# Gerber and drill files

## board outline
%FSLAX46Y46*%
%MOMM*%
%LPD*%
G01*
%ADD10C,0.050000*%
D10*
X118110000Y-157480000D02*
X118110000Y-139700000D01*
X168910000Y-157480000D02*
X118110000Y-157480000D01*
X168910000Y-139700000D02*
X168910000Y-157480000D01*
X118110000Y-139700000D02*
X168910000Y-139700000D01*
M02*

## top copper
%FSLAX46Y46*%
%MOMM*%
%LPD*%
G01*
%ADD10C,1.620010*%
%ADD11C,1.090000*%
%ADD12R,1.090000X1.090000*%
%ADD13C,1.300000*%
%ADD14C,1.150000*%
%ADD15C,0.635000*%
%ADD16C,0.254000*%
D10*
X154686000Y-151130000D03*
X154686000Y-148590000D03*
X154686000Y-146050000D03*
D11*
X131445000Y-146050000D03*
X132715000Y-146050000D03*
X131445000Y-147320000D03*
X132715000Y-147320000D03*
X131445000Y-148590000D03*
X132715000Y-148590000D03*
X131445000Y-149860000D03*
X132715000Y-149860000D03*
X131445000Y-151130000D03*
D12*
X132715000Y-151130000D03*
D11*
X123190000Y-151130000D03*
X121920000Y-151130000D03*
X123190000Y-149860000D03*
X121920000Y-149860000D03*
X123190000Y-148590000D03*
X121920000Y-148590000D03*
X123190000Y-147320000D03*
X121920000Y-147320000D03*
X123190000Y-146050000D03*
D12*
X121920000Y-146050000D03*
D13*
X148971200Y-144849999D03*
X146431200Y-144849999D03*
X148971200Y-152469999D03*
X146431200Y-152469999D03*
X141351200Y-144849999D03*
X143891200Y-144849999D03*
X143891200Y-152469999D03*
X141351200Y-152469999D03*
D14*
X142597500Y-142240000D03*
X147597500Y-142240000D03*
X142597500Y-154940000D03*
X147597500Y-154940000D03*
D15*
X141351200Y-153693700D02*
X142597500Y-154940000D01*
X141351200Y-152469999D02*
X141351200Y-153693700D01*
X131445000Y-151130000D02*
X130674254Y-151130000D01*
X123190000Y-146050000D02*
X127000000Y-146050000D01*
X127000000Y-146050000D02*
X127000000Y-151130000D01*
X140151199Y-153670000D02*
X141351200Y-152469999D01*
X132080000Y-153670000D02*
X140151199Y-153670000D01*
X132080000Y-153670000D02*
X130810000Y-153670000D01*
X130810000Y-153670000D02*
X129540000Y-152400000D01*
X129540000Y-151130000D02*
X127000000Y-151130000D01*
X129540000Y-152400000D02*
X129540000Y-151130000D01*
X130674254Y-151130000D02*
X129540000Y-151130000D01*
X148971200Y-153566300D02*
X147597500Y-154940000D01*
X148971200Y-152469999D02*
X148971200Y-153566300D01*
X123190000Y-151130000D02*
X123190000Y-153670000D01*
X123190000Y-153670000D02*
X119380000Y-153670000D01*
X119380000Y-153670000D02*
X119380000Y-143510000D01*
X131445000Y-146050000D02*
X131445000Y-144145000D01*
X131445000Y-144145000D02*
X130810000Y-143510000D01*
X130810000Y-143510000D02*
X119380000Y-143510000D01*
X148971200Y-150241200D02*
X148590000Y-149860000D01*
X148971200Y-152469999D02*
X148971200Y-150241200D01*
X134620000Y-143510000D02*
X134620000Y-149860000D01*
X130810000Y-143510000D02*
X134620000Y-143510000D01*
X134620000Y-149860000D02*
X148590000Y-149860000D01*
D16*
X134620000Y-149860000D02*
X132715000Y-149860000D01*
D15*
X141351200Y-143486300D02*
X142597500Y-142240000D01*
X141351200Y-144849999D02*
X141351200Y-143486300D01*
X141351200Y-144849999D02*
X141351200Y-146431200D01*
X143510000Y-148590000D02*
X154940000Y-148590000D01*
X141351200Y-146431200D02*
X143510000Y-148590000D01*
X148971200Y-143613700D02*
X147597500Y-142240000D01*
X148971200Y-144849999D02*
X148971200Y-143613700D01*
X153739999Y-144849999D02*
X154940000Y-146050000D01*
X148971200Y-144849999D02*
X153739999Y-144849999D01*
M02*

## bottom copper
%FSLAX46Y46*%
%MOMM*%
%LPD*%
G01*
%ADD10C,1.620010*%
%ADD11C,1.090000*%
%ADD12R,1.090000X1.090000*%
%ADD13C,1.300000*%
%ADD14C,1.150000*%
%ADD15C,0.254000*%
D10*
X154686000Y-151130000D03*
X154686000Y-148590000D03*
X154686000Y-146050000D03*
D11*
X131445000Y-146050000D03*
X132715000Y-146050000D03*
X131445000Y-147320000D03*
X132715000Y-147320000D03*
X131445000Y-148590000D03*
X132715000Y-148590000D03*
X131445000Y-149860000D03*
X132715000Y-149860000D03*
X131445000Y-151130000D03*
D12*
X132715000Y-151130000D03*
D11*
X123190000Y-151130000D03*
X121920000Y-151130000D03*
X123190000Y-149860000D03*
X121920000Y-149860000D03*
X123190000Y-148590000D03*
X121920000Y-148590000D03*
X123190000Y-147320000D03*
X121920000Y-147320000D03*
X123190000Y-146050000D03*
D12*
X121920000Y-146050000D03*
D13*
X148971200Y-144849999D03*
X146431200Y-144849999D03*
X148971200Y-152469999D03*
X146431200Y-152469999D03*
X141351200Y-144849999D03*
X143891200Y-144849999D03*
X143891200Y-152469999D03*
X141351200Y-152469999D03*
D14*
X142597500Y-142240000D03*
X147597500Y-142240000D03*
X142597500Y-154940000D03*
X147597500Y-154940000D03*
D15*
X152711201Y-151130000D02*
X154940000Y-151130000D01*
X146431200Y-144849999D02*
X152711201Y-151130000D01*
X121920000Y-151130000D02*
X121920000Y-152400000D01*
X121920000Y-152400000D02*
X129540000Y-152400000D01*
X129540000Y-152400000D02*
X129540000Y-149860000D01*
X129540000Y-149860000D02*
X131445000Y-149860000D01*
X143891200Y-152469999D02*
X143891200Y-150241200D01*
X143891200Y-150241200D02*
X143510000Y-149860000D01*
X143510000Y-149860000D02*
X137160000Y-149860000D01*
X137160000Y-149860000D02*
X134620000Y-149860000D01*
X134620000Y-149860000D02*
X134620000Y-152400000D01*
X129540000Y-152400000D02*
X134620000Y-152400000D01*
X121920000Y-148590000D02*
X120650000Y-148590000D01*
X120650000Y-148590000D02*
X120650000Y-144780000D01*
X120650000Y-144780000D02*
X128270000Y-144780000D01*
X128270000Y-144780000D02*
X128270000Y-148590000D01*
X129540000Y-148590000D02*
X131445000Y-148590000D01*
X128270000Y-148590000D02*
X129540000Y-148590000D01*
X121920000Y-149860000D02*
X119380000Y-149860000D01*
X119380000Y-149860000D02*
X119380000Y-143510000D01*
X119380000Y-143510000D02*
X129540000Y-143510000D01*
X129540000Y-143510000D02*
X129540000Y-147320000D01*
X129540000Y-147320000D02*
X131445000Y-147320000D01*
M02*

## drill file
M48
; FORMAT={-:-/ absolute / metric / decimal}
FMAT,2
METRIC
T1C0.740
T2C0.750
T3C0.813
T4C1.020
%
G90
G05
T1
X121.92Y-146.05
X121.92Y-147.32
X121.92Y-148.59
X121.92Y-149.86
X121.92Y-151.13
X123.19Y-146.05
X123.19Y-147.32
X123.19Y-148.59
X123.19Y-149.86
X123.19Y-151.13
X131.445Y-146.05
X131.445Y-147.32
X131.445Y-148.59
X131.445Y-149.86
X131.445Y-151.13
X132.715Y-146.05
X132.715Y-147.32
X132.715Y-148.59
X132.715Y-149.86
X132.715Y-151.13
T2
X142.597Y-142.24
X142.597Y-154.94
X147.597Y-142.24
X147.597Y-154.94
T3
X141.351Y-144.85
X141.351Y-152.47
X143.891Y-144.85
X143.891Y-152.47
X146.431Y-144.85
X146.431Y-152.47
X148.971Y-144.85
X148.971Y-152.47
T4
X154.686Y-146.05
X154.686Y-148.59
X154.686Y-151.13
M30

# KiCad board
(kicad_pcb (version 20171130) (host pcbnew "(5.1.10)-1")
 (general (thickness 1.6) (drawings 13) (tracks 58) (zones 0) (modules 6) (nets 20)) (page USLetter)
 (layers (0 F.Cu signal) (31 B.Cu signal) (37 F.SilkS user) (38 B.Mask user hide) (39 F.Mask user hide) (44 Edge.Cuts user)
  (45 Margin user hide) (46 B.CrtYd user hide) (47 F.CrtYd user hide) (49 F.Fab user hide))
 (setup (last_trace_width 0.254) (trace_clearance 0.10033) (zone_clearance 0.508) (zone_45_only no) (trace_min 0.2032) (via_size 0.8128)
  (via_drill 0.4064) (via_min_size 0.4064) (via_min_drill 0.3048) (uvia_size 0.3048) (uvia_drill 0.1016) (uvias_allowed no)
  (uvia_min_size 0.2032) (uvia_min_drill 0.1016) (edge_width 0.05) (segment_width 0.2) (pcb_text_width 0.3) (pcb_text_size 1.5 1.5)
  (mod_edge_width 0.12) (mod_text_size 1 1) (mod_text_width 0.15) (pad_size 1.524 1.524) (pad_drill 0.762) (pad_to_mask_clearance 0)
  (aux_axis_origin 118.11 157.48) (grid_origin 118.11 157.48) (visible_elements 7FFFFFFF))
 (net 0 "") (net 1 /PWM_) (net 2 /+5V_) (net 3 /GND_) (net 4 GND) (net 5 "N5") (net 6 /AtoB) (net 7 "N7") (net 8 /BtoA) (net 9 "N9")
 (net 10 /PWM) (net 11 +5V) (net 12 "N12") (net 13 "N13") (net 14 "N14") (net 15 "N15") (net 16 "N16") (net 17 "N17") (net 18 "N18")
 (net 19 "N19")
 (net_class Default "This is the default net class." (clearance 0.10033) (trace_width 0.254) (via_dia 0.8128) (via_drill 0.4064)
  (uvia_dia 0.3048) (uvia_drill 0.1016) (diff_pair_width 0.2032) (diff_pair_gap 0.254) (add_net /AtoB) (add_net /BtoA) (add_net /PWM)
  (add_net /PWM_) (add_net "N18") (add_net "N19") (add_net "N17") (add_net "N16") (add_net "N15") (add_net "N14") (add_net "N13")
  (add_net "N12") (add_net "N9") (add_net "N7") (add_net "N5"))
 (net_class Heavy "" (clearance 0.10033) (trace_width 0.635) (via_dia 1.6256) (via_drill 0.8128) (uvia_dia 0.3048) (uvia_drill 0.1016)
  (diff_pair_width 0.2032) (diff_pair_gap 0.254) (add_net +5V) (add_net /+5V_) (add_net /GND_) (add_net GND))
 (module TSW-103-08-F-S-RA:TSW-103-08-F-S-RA (layer F.Cu) (at 157.48 148.59 270)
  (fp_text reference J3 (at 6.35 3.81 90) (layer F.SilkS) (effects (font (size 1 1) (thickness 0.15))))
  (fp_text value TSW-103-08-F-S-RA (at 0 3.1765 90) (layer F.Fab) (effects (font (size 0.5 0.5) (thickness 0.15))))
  (pad 3 thru_hole circle (at 2.54 2.794 270) (size 1.62001 1.62001) (drill 1.01999) (layers *.Cu) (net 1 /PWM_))
  (pad 2 thru_hole circle (at 0 2.794 270) (size 1.62001 1.62001) (drill 1.01999) (layers *.Cu) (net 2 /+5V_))
  (pad 1 thru_hole circle (at -2.54 2.794 270) (size 1.62001 1.62001) (drill 1.01999) (layers *.Cu) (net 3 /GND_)))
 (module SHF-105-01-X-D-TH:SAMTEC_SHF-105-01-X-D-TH (layer F.Cu) (at 132.08 148.59 90)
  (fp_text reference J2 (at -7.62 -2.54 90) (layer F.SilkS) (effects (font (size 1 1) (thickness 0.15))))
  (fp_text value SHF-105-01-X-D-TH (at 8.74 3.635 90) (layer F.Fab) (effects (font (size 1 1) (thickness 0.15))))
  (pad 10 thru_hole circle (at 2.54 -0.635 90) (size 1.09 1.09) (drill 0.74) (layers *.Cu *.Mask) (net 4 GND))
  (pad 09 thru_hole circle (at 2.54 0.635 90) (size 1.09 1.09) (drill 0.74) (layers *.Cu *.Mask) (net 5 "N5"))
  (pad 08 thru_hole circle (at 1.27 -0.635 90) (size 1.09 1.09) (drill 0.74) (layers *.Cu *.Mask) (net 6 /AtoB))
  (pad 07 thru_hole circle (at 1.27 0.635 90) (size 1.09 1.09) (drill 0.74) (layers *.Cu *.Mask) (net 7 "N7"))
  (pad 06 thru_hole circle (at 0 -0.635 90) (size 1.09 1.09) (drill 0.74) (layers *.Cu *.Mask) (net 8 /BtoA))
  (pad 05 thru_hole circle (at 0 0.635 90) (size 1.09 1.09) (drill 0.74) (layers *.Cu *.Mask) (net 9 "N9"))
  (pad 04 thru_hole circle (at -1.27 -0.635 90) (size 1.09 1.09) (drill 0.74) (layers *.Cu *.Mask) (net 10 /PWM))
  (pad 03 thru_hole circle (at -1.27 0.635 90) (size 1.09 1.09) (drill 0.74) (layers *.Cu *.Mask) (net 4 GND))
  (pad 02 thru_hole circle (at -2.54 -0.635 90) (size 1.09 1.09) (drill 0.74) (layers *.Cu *.Mask) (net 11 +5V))
  (pad 01 thru_hole rect (at -2.54 0.635 90) (size 1.09 1.09) (drill 0.74) (layers *.Cu *.Mask) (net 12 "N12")))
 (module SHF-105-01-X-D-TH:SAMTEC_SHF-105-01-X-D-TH (layer F.Cu) (at 122.555 148.59 270)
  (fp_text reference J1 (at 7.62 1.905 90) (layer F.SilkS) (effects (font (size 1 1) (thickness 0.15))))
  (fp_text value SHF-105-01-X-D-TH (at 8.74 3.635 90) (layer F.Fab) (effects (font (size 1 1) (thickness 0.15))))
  (pad 10 thru_hole circle (at 2.54 -0.635 270) (size 1.09 1.09) (drill 0.74) (layers *.Cu *.Mask) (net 4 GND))
  (pad 09 thru_hole circle (at 2.54 0.635 270) (size 1.09 1.09) (drill 0.74) (layers *.Cu *.Mask) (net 10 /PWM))
  (pad 08 thru_hole circle (at 1.27 -0.635 270) (size 1.09 1.09) (drill 0.74) (layers *.Cu *.Mask) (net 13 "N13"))
  (pad 07 thru_hole circle (at 1.27 0.635 270) (size 1.09 1.09) (drill 0.74) (layers *.Cu *.Mask) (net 6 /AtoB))
  (pad 06 thru_hole circle (at 0 -0.635 270) (size 1.09 1.09) (drill 0.74) (layers *.Cu *.Mask) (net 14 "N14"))
  (pad 05 thru_hole circle (at 0 0.635 270) (size 1.09 1.09) (drill 0.74) (layers *.Cu *.Mask) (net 8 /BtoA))
  (pad 04 thru_hole circle (at -1.27 -0.635 270) (size 1.09 1.09) (drill 0.74) (layers *.Cu *.Mask) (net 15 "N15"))
  (pad 03 thru_hole circle (at -1.27 0.635 270) (size 1.09 1.09) (drill 0.74) (layers *.Cu *.Mask) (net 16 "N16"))
  (pad 02 thru_hole circle (at -2.54 -0.635 270) (size 1.09 1.09) (drill 0.74) (layers *.Cu *.Mask) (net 11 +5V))
  (pad 01 thru_hole rect (at -2.54 0.635 270) (size 1.09 1.09) (drill 0.74) (layers *.Cu *.Mask) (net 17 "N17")))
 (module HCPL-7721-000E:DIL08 (layer F.Cu) (at 145.1612 148.659999)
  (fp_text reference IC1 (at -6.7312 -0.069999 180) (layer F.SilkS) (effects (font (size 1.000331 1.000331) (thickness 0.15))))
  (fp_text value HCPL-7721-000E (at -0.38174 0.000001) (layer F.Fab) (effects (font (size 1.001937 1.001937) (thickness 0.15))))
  (pad 5 thru_hole circle (at 3.81 -3.81) (size 1.3 1.3) (drill 0.8128) (layers *.Cu *.Mask) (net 3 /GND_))
  (pad 6 thru_hole circle (at 1.27 -3.81) (size 1.3 1.3) (drill 0.8128) (layers *.Cu *.Mask) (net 1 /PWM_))
  (pad 4 thru_hole circle (at 3.81 3.81) (size 1.3 1.3) (drill 0.8128) (layers *.Cu *.Mask) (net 4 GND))
  (pad 3 thru_hole circle (at 1.27 3.81) (size 1.3 1.3) (drill 0.8128) (layers *.Cu *.Mask) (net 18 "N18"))
  (pad 8 thru_hole circle (at -3.81 -3.81) (size 1.3 1.3) (drill 0.8128) (layers *.Cu *.Mask) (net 2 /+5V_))
  (pad 7 thru_hole circle (at -1.27 -3.81) (size 1.3 1.3) (drill 0.8128) (layers *.Cu *.Mask) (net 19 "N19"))
  (pad 2 thru_hole circle (at -1.27 3.81) (size 1.3 1.3) (drill 0.8128) (layers *.Cu *.Mask) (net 10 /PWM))
  (pad 1 thru_hole circle (at -3.81 3.81) (size 1.3 1.3) (drill 0.8128) (layers *.Cu *.Mask) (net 11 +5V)))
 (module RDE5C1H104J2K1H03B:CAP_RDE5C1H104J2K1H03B (layer F.Cu) (at 145.0975 142.24 180)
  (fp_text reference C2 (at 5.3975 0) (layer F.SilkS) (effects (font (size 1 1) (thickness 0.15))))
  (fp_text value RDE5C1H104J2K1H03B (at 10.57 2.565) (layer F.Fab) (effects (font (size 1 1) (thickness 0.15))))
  (pad 2 thru_hole circle (at 2.5 0 180) (size 1.15 1.15) (drill 0.75) (layers *.Cu *.Mask) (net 2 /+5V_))
  (pad 1 thru_hole circle (at -2.5 0 180) (size 1.15 1.15) (drill 0.75) (layers *.Cu *.Mask) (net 3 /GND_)))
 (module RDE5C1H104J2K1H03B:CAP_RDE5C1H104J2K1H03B (layer F.Cu) (at 145.0975 154.94 180)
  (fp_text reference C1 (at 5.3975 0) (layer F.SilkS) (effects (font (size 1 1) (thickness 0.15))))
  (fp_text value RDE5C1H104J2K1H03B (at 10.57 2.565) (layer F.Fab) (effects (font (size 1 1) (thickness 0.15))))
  (pad 2 thru_hole circle (at 2.5 0 180) (size 1.15 1.15) (drill 0.75) (layers *.Cu *.Mask) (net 11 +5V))
  (pad 1 thru_hole circle (at -2.5 0 180) (size 1.15 1.15) (drill 0.75) (layers *.Cu *.Mask) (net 4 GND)))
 (gr_line (start 118.11 157.48) (end 118.11 139.7) (layer Edge.Cuts) (width 0.05))
 (gr_line (start 168.91 157.48) (end 118.11 157.48) (layer Edge.Cuts) (width 0.05))
 (gr_line (start 168.91 139.7) (end 168.91 157.48) (layer Edge.Cuts) (width 0.05))
 (gr_line (start 118.11 139.7) (end 168.91 139.7) (layer Edge.Cuts) (width 0.05))
 (segment (start 141.3512 153.6937) (end 142.5975 154.94) (width 0.635) (layer F.Cu) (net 11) (status 20))
 (segment (start 141.3512 152.469999) (end 141.3512 153.6937) (width 0.635) (layer F.Cu) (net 11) (status 10))
 (segment (start 131.445 151.13) (end 130.674254 151.13) (width 0.635) (layer F.Cu) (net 11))
 (segment (start 123.19 146.05) (end 127 146.05) (width 0.635) (layer F.Cu) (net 11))
 (segment (start 127 146.05) (end 127 151.13) (width 0.635) (layer F.Cu) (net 11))
 (segment (start 140.151199 153.67) (end 141.3512 152.469999) (width 0.635) (layer F.Cu) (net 11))
 (segment (start 132.08 153.67) (end 140.151199 153.67) (width 0.635) (layer F.Cu) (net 11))
 (segment (start 132.08 153.67) (end 130.81 153.67) (width 0.635) (layer F.Cu) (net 11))
 (segment (start 130.81 153.67) (end 129.54 152.4) (width 0.635) (layer F.Cu) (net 11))
 (segment (start 129.54 151.13) (end 127 151.13) (width 0.635) (layer F.Cu) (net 11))
 (segment (start 129.54 152.4) (end 129.54 151.13) (width 0.635) (layer F.Cu) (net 11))
 (segment (start 130.674254 151.13) (end 129.54 151.13) (width 0.635) (layer F.Cu) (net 11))
 (segment (start 148.9712 153.5663) (end 147.5975 154.94) (width 0.635) (layer F.Cu) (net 4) (status 20))
 (segment (start 148.9712 152.469999) (end 148.9712 153.5663) (width 0.635) (layer F.Cu) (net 4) (status 10))
 (segment (start 123.19 151.13) (end 123.19 153.67) (width 0.635) (layer F.Cu) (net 4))
 (segment (start 123.19 153.67) (end 119.38 153.67) (width 0.635) (layer F.Cu) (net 4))
 (segment (start 119.38 153.67) (end 119.38 143.51) (width 0.635) (layer F.Cu) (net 4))
 (segment (start 131.445 146.05) (end 131.445 144.145) (width 0.635) (layer F.Cu) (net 4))
 (segment (start 131.445 144.145) (end 130.81 143.51) (width 0.635) (layer F.Cu) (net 4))
 (segment (start 130.81 143.51) (end 119.38 143.51) (width 0.635) (layer F.Cu) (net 4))
 (segment (start 148.9712 150.2412) (end 148.59 149.86) (width 0.635) (layer F.Cu) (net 4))
 (segment (start 148.9712 152.469999) (end 148.9712 150.2412) (width 0.635) (layer F.Cu) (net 4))
 (segment (start 134.62 143.51) (end 134.62 149.86) (width 0.635) (layer F.Cu) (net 4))
 (segment (start 130.81 143.51) (end 134.62 143.51) (width 0.635) (layer F.Cu) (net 4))
 (segment (start 134.62 149.86) (end 148.59 149.86) (width 0.635) (layer F.Cu) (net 4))
 (segment (start 134.62 149.86) (end 132.715 149.86) (width 0.254) (layer F.Cu) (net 4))
 (segment (start 141.3512 143.4863) (end 142.5975 142.24) (width 0.635) (layer F.Cu) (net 2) (status 20))
 (segment (start 141.3512 144.849999) (end 141.3512 143.4863) (width 0.635) (layer F.Cu) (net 2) (status 10))
 (segment (start 141.3512 144.849999) (end 141.3512 146.4312) (width 0.635) (layer F.Cu) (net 2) (status 10))
 (segment (start 143.51 148.59) (end 154.94 148.59) (width 0.635) (layer F.Cu) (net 2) (status 20))
 (segment (start 141.3512 146.4312) (end 143.51 148.59) (width 0.635) (layer F.Cu) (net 2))
 (segment (start 148.9712 143.6137) (end 147.5975 142.24) (width 0.635) (layer F.Cu) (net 3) (status 20))
 (segment (start 148.9712 144.849999) (end 148.9712 143.6137) (width 0.635) (layer F.Cu) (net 3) (status 10))
 (segment (start 153.739999 144.849999) (end 154.94 146.05) (width 0.635) (layer F.Cu) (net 3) (status 20))
 (segment (start 148.9712 144.849999) (end 153.739999 144.849999) (width 0.635) (layer F.Cu) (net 3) (status 10))
 (segment (start 152.711201 151.13) (end 154.94 151.13) (width 0.254) (layer B.Cu) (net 1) (status 20))
 (segment (start 146.4312 144.849999) (end 152.711201 151.13) (width 0.254) (layer B.Cu) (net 1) (status 10))
 (segment (start 121.92 151.13) (end 121.92 152.4) (width 0.254) (layer B.Cu) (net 10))
 (segment (start 121.92 152.4) (end 129.54 152.4) (width 0.254) (layer B.Cu) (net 10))
 (segment (start 129.54 152.4) (end 129.54 149.86) (width 0.254) (layer B.Cu) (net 10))
 (segment (start 129.54 149.86) (end 131.445 149.86) (width 0.254) (layer B.Cu) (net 10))
 (segment (start 143.8912 152.469999) (end 143.8912 150.2412) (width 0.254) (layer B.Cu) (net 10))
 (segment (start 143.8912 150.2412) (end 143.51 149.86) (width 0.254) (layer B.Cu) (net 10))
 (segment (start 143.51 149.86) (end 137.16 149.86) (width 0.254) (layer B.Cu) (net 10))
 (segment (start 137.16 149.86) (end 134.62 149.86) (width 0.254) (layer B.Cu) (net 10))
 (segment (start 134.62 149.86) (end 134.62 152.4) (width 0.254) (layer B.Cu) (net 10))
 (segment (start 129.54 152.4) (end 134.62 152.4) (width 0.254) (layer B.Cu) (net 10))
 (segment (start 121.92 148.59) (end 120.65 148.59) (width 0.254) (layer B.Cu) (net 8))
 (segment (start 120.65 148.59) (end 120.65 144.78) (width 0.254) (layer B.Cu) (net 8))
 (segment (start 120.65 144.78) (end 128.27 144.78) (width 0.254) (layer B.Cu) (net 8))
 (segment (start 128.27 144.78) (end 128.27 148.59) (width 0.254) (layer B.Cu) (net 8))
 (segment (start 129.54 148.59) (end 131.445 148.59) (width 0.254) (layer B.Cu) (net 8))
 (segment (start 128.27 148.59) (end 129.54 148.59) (width 0.254) (layer B.Cu) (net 8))
 (segment (start 121.92 149.86) (end 119.38 149.86) (width 0.254) (layer B.Cu) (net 6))
 (segment (start 119.38 149.86) (end 119.38 143.51) (width 0.254) (layer B.Cu) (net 6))
 (segment (start 119.38 143.51) (end 129.54 143.51) (width 0.254) (layer B.Cu) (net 6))
 (segment (start 129.54 143.51) (end 129.54 147.32) (width 0.254) (layer B.Cu) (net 6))
 (segment (start 129.54 147.32) (end 131.445 147.32) (width 0.254) (layer B.Cu) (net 6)))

